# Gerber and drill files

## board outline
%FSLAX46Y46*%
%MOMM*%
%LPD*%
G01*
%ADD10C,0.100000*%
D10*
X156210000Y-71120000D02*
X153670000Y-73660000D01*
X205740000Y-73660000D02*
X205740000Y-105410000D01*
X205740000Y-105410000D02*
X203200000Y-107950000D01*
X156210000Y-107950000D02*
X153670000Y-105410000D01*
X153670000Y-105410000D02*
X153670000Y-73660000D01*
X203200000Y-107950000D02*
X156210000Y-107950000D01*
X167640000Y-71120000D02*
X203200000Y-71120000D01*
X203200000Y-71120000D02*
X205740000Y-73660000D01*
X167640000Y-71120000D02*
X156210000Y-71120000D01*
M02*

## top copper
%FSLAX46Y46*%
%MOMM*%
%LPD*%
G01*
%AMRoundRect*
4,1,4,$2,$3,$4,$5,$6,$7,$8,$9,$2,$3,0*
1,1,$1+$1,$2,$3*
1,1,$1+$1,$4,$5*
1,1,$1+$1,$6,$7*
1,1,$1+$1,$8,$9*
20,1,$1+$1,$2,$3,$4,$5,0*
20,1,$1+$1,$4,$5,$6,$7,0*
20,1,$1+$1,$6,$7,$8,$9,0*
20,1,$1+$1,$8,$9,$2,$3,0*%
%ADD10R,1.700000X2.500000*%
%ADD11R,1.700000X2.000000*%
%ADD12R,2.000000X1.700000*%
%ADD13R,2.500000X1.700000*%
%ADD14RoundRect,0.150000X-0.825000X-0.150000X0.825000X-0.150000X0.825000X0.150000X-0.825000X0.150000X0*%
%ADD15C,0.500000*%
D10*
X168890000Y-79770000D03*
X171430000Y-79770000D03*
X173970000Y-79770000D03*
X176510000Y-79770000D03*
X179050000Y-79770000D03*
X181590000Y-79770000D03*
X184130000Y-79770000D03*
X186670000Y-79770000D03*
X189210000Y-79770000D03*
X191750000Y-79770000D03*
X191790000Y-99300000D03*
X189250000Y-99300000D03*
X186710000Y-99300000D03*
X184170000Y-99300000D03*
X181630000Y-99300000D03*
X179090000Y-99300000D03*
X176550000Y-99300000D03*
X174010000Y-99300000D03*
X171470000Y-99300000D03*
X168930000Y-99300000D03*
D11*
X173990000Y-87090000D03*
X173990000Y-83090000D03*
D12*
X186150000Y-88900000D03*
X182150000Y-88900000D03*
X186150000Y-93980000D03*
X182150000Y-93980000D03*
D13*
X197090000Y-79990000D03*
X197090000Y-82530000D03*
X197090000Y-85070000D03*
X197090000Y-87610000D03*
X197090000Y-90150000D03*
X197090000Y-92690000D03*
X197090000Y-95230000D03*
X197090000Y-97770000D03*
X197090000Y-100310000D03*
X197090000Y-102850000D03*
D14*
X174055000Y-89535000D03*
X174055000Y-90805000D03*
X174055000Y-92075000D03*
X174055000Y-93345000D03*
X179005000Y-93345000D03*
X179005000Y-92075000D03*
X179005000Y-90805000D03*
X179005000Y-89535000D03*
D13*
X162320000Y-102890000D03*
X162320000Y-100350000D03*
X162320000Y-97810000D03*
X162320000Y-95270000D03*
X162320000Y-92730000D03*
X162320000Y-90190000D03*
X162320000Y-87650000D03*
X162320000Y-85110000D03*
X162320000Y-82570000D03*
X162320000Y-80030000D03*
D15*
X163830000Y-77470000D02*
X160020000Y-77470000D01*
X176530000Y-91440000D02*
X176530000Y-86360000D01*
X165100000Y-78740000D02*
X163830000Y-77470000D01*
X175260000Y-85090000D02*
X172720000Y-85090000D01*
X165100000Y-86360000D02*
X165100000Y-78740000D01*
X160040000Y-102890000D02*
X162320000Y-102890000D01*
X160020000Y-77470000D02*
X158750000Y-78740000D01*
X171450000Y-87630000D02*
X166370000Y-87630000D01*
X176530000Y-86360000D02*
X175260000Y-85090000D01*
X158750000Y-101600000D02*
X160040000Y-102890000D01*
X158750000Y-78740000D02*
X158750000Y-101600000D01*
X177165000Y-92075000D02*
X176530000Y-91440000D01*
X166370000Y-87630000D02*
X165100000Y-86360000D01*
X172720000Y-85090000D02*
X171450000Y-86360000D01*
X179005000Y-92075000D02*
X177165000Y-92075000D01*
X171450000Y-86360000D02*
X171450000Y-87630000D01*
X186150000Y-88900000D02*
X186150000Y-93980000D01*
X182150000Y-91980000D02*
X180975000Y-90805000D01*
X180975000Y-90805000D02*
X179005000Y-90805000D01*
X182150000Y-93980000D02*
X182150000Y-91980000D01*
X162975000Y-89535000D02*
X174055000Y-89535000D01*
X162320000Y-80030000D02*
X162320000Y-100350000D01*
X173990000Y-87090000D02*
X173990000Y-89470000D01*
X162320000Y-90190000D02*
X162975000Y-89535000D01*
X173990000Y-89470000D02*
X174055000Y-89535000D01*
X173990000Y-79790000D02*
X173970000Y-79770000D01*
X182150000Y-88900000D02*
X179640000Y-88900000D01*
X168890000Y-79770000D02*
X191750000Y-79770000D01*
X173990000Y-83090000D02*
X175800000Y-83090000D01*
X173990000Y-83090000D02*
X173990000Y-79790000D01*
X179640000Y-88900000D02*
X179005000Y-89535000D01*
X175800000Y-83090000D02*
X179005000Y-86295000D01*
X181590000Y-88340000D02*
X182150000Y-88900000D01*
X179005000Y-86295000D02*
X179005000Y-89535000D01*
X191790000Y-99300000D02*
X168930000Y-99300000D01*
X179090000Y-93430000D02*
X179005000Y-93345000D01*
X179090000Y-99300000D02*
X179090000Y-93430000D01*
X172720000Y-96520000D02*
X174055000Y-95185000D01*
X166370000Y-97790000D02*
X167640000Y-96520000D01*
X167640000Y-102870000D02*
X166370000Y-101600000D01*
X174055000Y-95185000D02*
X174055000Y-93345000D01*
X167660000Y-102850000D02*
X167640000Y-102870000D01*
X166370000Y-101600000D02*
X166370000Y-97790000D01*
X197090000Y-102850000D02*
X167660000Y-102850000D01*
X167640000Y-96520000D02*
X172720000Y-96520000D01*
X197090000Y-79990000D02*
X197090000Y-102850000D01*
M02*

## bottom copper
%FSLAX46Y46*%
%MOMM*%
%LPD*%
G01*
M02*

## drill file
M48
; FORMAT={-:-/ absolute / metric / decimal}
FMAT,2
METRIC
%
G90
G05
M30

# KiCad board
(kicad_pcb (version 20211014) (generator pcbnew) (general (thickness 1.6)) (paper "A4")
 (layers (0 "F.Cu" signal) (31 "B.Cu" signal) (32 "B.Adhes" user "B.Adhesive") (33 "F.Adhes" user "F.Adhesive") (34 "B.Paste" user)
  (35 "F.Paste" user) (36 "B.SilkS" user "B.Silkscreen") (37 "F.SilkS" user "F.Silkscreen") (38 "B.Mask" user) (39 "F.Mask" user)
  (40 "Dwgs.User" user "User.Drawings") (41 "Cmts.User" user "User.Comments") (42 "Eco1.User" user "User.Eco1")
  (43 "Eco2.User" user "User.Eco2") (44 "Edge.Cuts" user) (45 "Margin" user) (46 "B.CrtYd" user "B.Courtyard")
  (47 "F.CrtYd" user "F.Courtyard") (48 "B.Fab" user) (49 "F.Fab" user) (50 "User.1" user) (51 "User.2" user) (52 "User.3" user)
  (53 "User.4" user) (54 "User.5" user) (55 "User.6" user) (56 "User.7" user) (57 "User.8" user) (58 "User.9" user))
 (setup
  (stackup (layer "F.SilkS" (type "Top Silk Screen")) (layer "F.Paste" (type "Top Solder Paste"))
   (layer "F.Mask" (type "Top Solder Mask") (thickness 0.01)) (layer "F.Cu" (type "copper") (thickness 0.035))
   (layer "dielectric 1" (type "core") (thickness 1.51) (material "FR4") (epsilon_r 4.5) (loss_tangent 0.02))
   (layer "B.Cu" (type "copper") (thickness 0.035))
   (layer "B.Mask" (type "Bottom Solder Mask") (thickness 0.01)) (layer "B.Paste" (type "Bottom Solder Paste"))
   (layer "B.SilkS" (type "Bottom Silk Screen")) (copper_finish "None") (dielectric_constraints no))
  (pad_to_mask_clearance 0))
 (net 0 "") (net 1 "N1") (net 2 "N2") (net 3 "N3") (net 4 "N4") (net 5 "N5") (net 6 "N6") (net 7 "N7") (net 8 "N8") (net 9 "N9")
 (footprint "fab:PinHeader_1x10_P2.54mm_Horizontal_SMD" (layer "F.Cu") (at 168.89 79.77 90)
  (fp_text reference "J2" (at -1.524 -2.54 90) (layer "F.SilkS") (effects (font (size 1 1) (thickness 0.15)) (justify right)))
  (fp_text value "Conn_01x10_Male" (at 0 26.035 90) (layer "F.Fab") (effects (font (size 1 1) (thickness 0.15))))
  (pad "1" smd rect locked (at 0 0 90) (size 2.5 1.7) (layers "F.Cu" "F.Paste" "F.Mask") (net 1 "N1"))
  (pad "2" smd rect locked (at 0 2.54 90) (size 2.5 1.7) (layers "F.Cu" "F.Paste" "F.Mask") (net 1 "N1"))
  (pad "3" smd rect locked (at 0 5.08 90) (size 2.5 1.7) (layers "F.Cu" "F.Paste" "F.Mask") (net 1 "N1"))
  (pad "4" smd rect locked (at 0 7.62 90) (size 2.5 1.7) (layers "F.Cu" "F.Paste" "F.Mask") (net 1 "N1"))
  (pad "5" smd rect locked (at 0 10.16 90) (size 2.5 1.7) (layers "F.Cu" "F.Paste" "F.Mask") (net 1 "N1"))
  (pad "6" smd rect locked (at 0 12.7 90) (size 2.5 1.7) (layers "F.Cu" "F.Paste" "F.Mask") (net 1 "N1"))
  (pad "7" smd rect locked (at 0 15.24 90) (size 2.5 1.7) (layers "F.Cu" "F.Paste" "F.Mask") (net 1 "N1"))
  (pad "8" smd rect locked (at 0 17.78 90) (size 2.5 1.7) (layers "F.Cu" "F.Paste" "F.Mask") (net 1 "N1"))
  (pad "9" smd rect locked (at 0 20.32 90) (size 2.5 1.7) (layers "F.Cu" "F.Paste" "F.Mask") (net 1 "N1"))
  (pad "10" smd rect locked (at 0 22.86 90) (size 2.5 1.7) (layers "F.Cu" "F.Paste" "F.Mask") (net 1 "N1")))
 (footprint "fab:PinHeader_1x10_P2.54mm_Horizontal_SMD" (layer "F.Cu") (at 191.79 99.3 -90)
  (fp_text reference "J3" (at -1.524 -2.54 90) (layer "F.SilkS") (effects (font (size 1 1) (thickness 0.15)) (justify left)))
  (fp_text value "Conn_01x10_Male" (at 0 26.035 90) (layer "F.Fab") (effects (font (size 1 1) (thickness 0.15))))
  (pad "1" smd rect locked (at 0 0 270) (size 2.5 1.7) (layers "F.Cu" "F.Paste" "F.Mask") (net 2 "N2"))
  (pad "2" smd rect locked (at 0 2.54 270) (size 2.5 1.7) (layers "F.Cu" "F.Paste" "F.Mask") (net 2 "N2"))
  (pad "3" smd rect locked (at 0 5.08 270) (size 2.5 1.7) (layers "F.Cu" "F.Paste" "F.Mask") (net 2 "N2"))
  (pad "4" smd rect locked (at 0 7.62 270) (size 2.5 1.7) (layers "F.Cu" "F.Paste" "F.Mask") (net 2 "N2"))
  (pad "5" smd rect locked (at 0 10.16 270) (size 2.5 1.7) (layers "F.Cu" "F.Paste" "F.Mask") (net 2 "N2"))
  (pad "6" smd rect locked (at 0 12.7 270) (size 2.5 1.7) (layers "F.Cu" "F.Paste" "F.Mask") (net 2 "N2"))
  (pad "7" smd rect locked (at 0 15.24 270) (size 2.5 1.7) (layers "F.Cu" "F.Paste" "F.Mask") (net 2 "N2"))
  (pad "8" smd rect locked (at 0 17.78 270) (size 2.5 1.7) (layers "F.Cu" "F.Paste" "F.Mask") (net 2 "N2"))
  (pad "9" smd rect locked (at 0 20.32 270) (size 2.5 1.7) (layers "F.Cu" "F.Paste" "F.Mask") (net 2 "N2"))
  (pad "10" smd rect locked (at 0 22.86 270) (size 2.5 1.7) (layers "F.Cu" "F.Paste" "F.Mask") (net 2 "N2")))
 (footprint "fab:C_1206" (layer "F.Cu") (at 173.99 85.09 90)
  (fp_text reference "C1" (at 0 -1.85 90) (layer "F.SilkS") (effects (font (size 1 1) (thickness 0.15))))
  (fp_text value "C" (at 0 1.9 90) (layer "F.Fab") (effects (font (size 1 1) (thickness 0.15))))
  (pad "1" smd rect locked (at -2 0 90) (size 2 1.7) (layers "F.Cu" "F.Paste" "F.Mask") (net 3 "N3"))
  (pad "2" smd rect locked (at 2 0 90) (size 2 1.7) (layers "F.Cu" "F.Paste" "F.Mask") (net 1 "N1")))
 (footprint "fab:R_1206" (layer "F.Cu") (at 184.15 88.9 180)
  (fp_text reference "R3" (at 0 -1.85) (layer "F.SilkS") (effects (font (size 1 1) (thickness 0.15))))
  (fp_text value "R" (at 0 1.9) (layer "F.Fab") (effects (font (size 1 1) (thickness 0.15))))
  (pad "1" smd rect locked (at -2 0 180) (size 2 1.7) (layers "F.Cu" "F.Paste" "F.Mask") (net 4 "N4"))
  (pad "2" smd rect locked (at 2 0 180) (size 2 1.7) (layers "F.Cu" "F.Paste" "F.Mask") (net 1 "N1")))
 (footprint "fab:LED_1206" (layer "F.Cu") (at 184.15 93.98 180)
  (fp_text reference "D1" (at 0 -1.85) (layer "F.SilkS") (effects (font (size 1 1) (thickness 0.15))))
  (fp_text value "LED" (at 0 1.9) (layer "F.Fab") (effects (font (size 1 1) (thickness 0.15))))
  (pad "1" smd rect locked (at -2 0 180) (size 2 1.7) (layers "F.Cu" "F.Paste" "F.Mask") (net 4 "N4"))
  (pad "2" smd rect locked (at 2 0 180) (size 2 1.7) (layers "F.Cu" "F.Paste" "F.Mask") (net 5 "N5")))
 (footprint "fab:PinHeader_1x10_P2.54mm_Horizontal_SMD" (layer "F.Cu") (at 197.09 79.99)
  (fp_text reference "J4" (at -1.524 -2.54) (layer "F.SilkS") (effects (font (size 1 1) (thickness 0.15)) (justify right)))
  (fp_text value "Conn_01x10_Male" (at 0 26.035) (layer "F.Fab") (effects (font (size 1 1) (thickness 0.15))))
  (pad "1" smd rect locked (at 0 0) (size 2.5 1.7) (layers "F.Cu" "F.Paste" "F.Mask") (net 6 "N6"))
  (pad "2" smd rect locked (at 0 2.54) (size 2.5 1.7) (layers "F.Cu" "F.Paste" "F.Mask") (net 6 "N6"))
  (pad "3" smd rect locked (at 0 5.08) (size 2.5 1.7) (layers "F.Cu" "F.Paste" "F.Mask") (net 6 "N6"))
  (pad "4" smd rect locked (at 0 7.62) (size 2.5 1.7) (layers "F.Cu" "F.Paste" "F.Mask") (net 6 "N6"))
  (pad "5" smd rect locked (at 0 10.16) (size 2.5 1.7) (layers "F.Cu" "F.Paste" "F.Mask") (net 6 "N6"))
  (pad "6" smd rect locked (at 0 12.7) (size 2.5 1.7) (layers "F.Cu" "F.Paste" "F.Mask") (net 6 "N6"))
  (pad "7" smd rect locked (at 0 15.24) (size 2.5 1.7) (layers "F.Cu" "F.Paste" "F.Mask") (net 6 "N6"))
  (pad "8" smd rect locked (at 0 17.78) (size 2.5 1.7) (layers "F.Cu" "F.Paste" "F.Mask") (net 6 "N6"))
  (pad "9" smd rect locked (at 0 20.32) (size 2.5 1.7) (layers "F.Cu" "F.Paste" "F.Mask") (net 6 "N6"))
  (pad "10" smd rect locked (at 0 22.86) (size 2.5 1.7) (layers "F.Cu" "F.Paste" "F.Mask") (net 6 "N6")))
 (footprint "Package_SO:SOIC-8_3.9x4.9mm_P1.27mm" (layer "F.Cu") (at 176.53 91.44)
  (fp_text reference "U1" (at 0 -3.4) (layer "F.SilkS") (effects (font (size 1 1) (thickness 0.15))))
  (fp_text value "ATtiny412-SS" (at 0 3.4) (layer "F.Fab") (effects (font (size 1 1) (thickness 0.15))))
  (pad "1" smd roundrect (at -2.475 -1.905) (size 1.95 0.6) (layers "F.Cu" "F.Paste" "F.Mask") (roundrect_rratio 0.25) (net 3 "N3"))
  (pad "2" smd roundrect (at -2.475 -0.635) (size 1.95 0.6) (layers "F.Cu" "F.Paste" "F.Mask") (roundrect_rratio 0.25) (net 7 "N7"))
  (pad "3" smd roundrect (at -2.475 0.635) (size 1.95 0.6) (layers "F.Cu" "F.Paste" "F.Mask") (roundrect_rratio 0.25) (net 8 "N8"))
  (pad "4" smd roundrect (at -2.475 1.905) (size 1.95 0.6) (layers "F.Cu" "F.Paste" "F.Mask") (roundrect_rratio 0.25) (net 6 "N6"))
  (pad "5" smd roundrect (at 2.475 1.905) (size 1.95 0.6) (layers "F.Cu" "F.Paste" "F.Mask") (roundrect_rratio 0.25) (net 2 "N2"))
  (pad "6" smd roundrect (at 2.475 0.635) (size 1.95 0.6) (layers "F.Cu" "F.Paste" "F.Mask") (roundrect_rratio 0.25) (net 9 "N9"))
  (pad "7" smd roundrect (at 2.475 -0.635) (size 1.95 0.6) (layers "F.Cu" "F.Paste" "F.Mask") (roundrect_rratio 0.25) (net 5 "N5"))
  (pad "8" smd roundrect (at 2.475 -1.905) (size 1.95 0.6) (layers "F.Cu" "F.Paste" "F.Mask") (roundrect_rratio 0.25) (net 1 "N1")))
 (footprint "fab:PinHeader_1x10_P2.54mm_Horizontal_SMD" (layer "F.Cu") (at 162.32 102.89 180)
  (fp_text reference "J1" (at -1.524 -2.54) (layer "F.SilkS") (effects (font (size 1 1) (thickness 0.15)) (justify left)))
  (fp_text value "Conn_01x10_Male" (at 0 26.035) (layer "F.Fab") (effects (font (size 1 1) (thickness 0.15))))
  (pad "1" smd rect locked (at 0 0 180) (size 2.5 1.7) (layers "F.Cu" "F.Paste" "F.Mask") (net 9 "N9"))
  (pad "2" smd rect locked (at 0 2.54 180) (size 2.5 1.7) (layers "F.Cu" "F.Paste" "F.Mask") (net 3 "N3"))
  (pad "3" smd rect locked (at 0 5.08 180) (size 2.5 1.7) (layers "F.Cu" "F.Paste" "F.Mask") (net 3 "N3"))
  (pad "4" smd rect locked (at 0 7.62 180) (size 2.5 1.7) (layers "F.Cu" "F.Paste" "F.Mask") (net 3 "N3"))
  (pad "5" smd rect locked (at 0 10.16 180) (size 2.5 1.7) (layers "F.Cu" "F.Paste" "F.Mask") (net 3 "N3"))
  (pad "6" smd rect locked (at 0 12.7 180) (size 2.5 1.7) (layers "F.Cu" "F.Paste" "F.Mask") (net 3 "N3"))
  (pad "7" smd rect locked (at 0 15.24 180) (size 2.5 1.7) (layers "F.Cu" "F.Paste" "F.Mask") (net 3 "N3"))
  (pad "8" smd rect locked (at 0 17.78 180) (size 2.5 1.7) (layers "F.Cu" "F.Paste" "F.Mask") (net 3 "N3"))
  (pad "9" smd rect locked (at 0 20.32 180) (size 2.5 1.7) (layers "F.Cu" "F.Paste" "F.Mask") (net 3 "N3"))
  (pad "10" smd rect locked (at 0 22.86 180) (size 2.5 1.7) (layers "F.Cu" "F.Paste" "F.Mask") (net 3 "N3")))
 (gr_line (start 156.21 71.12) (end 153.67 73.66) (layer "Edge.Cuts") (width 0.1))
 (gr_line (start 205.74 73.66) (end 205.74 105.41) (layer "Edge.Cuts") (width 0.1))
 (gr_line (start 205.74 105.41) (end 203.2 107.95) (layer "Edge.Cuts") (width 0.1))
 (gr_line (start 156.21 107.95) (end 153.67 105.41) (layer "Edge.Cuts") (width 0.1))
 (gr_line (start 153.67 105.41) (end 153.67 73.66) (layer "Edge.Cuts") (width 0.1))
 (gr_line (start 203.2 107.95) (end 156.21 107.95) (layer "Edge.Cuts") (width 0.1))
 (gr_line (start 167.64 71.12) (end 203.2 71.12) (layer "Edge.Cuts") (width 0.1))
 (gr_line (start 203.2 71.12) (end 205.74 73.66) (layer "Edge.Cuts") (width 0.1))
 (gr_line (start 167.64 71.12) (end 156.21 71.12) (layer "Edge.Cuts") (width 0.1))
 (segment (start 163.83 77.47) (end 160.02 77.47) (width 0.5) (layer "F.Cu") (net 9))
 (segment (start 176.53 91.44) (end 176.53 86.36) (width 0.5) (layer "F.Cu") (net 9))
 (segment (start 165.1 78.74) (end 163.83 77.47) (width 0.5) (layer "F.Cu") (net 9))
 (segment (start 175.26 85.09) (end 172.72 85.09) (width 0.5) (layer "F.Cu") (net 9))
 (segment (start 165.1 86.36) (end 165.1 78.74) (width 0.5) (layer "F.Cu") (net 9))
 (segment (start 160.04 102.89) (end 162.32 102.89) (width 0.5) (layer "F.Cu") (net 9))
 (segment (start 160.02 77.47) (end 158.75 78.74) (width 0.5) (layer "F.Cu") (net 9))
 (segment (start 171.45 87.63) (end 166.37 87.63) (width 0.5) (layer "F.Cu") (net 9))
 (segment (start 176.53 86.36) (end 175.26 85.09) (width 0.5) (layer "F.Cu") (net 9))
 (segment (start 158.75 101.6) (end 160.04 102.89) (width 0.5) (layer "F.Cu") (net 9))
 (segment (start 158.75 78.74) (end 158.75 101.6) (width 0.5) (layer "F.Cu") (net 9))
 (segment (start 177.165 92.075) (end 176.53 91.44) (width 0.5) (layer "F.Cu") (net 9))
 (segment (start 166.37 87.63) (end 165.1 86.36) (width 0.5) (layer "F.Cu") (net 9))
 (segment (start 172.72 85.09) (end 171.45 86.36) (width 0.5) (layer "F.Cu") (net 9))
 (segment (start 179.005 92.075) (end 177.165 92.075) (width 0.5) (layer "F.Cu") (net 9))
 (segment (start 171.45 86.36) (end 171.45 87.63) (width 0.5) (layer "F.Cu") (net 9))
 (segment (start 186.15 88.9) (end 186.15 93.98) (width 0.5) (layer "F.Cu") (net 4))
 (segment (start 182.15 91.98) (end 180.975 90.805) (width 0.5) (layer "F.Cu") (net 5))
 (segment (start 180.975 90.805) (end 179.005 90.805) (width 0.5) (layer "F.Cu") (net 5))
 (segment (start 182.15 93.98) (end 182.15 91.98) (width 0.5) (layer "F.Cu") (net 5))
 (segment (start 162.975 89.535) (end 174.055 89.535) (width 0.5) (layer "F.Cu") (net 3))
 (segment (start 162.32 80.03) (end 162.32 100.35) (width 0.5) (layer "F.Cu") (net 3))
 (segment (start 173.99 87.09) (end 173.99 89.47) (width 0.5) (layer "F.Cu") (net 3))
 (segment (start 162.32 90.19) (end 162.975 89.535) (width 0.5) (layer "F.Cu") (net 3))
 (segment (start 173.99 89.47) (end 174.055 89.535) (width 0.5) (layer "F.Cu") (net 3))
 (segment (start 173.99 79.79) (end 173.97 79.77) (width 0.5) (layer "F.Cu") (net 1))
 (segment (start 182.15 88.9) (end 179.64 88.9) (width 0.5) (layer "F.Cu") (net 1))
 (segment (start 168.89 79.77) (end 191.75 79.77) (width 0.5) (layer "F.Cu") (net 1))
 (segment (start 173.99 83.09) (end 175.8 83.09) (width 0.5) (layer "F.Cu") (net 1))
 (segment (start 173.99 83.09) (end 173.99 79.79) (width 0.5) (layer "F.Cu") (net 1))
 (segment (start 179.64 88.9) (end 179.005 89.535) (width 0.5) (layer "F.Cu") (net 1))
 (segment (start 175.8 83.09) (end 179.005 86.295) (width 0.5) (layer "F.Cu") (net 1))
 (segment (start 181.59 88.34) (end 182.15 88.9) (width 0.5) (layer "F.Cu") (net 1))
 (segment (start 179.005 86.295) (end 179.005 89.535) (width 0.5) (layer "F.Cu") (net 1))
 (segment (start 191.79 99.3) (end 168.93 99.3) (width 0.5) (layer "F.Cu") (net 2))
 (segment (start 179.09 93.43) (end 179.005 93.345) (width 0.5) (layer "F.Cu") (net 2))
 (segment (start 179.09 99.3) (end 179.09 93.43) (width 0.5) (layer "F.Cu") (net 2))
 (segment (start 172.72 96.52) (end 174.055 95.185) (width 0.5) (layer "F.Cu") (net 6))
 (segment (start 166.37 97.79) (end 167.64 96.52) (width 0.5) (layer "F.Cu") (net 6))
 (segment (start 167.64 102.87) (end 166.37 101.6) (width 0.5) (layer "F.Cu") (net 6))
 (segment (start 174.055 95.185) (end 174.055 93.345) (width 0.5) (layer "F.Cu") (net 6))
 (segment (start 167.66 102.85) (end 167.64 102.87) (width 0.5) (layer "F.Cu") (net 6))
 (segment (start 166.37 101.6) (end 166.37 97.79) (width 0.5) (layer "F.Cu") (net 6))
 (segment (start 197.09 102.85) (end 167.66 102.85) (width 0.5) (layer "F.Cu") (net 6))
 (segment (start 167.64 96.52) (end 172.72 96.52) (width 0.5) (layer "F.Cu") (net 6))
 (segment (start 197.09 79.99) (end 197.09 102.85) (width 0.5) (layer "F.Cu") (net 6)))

